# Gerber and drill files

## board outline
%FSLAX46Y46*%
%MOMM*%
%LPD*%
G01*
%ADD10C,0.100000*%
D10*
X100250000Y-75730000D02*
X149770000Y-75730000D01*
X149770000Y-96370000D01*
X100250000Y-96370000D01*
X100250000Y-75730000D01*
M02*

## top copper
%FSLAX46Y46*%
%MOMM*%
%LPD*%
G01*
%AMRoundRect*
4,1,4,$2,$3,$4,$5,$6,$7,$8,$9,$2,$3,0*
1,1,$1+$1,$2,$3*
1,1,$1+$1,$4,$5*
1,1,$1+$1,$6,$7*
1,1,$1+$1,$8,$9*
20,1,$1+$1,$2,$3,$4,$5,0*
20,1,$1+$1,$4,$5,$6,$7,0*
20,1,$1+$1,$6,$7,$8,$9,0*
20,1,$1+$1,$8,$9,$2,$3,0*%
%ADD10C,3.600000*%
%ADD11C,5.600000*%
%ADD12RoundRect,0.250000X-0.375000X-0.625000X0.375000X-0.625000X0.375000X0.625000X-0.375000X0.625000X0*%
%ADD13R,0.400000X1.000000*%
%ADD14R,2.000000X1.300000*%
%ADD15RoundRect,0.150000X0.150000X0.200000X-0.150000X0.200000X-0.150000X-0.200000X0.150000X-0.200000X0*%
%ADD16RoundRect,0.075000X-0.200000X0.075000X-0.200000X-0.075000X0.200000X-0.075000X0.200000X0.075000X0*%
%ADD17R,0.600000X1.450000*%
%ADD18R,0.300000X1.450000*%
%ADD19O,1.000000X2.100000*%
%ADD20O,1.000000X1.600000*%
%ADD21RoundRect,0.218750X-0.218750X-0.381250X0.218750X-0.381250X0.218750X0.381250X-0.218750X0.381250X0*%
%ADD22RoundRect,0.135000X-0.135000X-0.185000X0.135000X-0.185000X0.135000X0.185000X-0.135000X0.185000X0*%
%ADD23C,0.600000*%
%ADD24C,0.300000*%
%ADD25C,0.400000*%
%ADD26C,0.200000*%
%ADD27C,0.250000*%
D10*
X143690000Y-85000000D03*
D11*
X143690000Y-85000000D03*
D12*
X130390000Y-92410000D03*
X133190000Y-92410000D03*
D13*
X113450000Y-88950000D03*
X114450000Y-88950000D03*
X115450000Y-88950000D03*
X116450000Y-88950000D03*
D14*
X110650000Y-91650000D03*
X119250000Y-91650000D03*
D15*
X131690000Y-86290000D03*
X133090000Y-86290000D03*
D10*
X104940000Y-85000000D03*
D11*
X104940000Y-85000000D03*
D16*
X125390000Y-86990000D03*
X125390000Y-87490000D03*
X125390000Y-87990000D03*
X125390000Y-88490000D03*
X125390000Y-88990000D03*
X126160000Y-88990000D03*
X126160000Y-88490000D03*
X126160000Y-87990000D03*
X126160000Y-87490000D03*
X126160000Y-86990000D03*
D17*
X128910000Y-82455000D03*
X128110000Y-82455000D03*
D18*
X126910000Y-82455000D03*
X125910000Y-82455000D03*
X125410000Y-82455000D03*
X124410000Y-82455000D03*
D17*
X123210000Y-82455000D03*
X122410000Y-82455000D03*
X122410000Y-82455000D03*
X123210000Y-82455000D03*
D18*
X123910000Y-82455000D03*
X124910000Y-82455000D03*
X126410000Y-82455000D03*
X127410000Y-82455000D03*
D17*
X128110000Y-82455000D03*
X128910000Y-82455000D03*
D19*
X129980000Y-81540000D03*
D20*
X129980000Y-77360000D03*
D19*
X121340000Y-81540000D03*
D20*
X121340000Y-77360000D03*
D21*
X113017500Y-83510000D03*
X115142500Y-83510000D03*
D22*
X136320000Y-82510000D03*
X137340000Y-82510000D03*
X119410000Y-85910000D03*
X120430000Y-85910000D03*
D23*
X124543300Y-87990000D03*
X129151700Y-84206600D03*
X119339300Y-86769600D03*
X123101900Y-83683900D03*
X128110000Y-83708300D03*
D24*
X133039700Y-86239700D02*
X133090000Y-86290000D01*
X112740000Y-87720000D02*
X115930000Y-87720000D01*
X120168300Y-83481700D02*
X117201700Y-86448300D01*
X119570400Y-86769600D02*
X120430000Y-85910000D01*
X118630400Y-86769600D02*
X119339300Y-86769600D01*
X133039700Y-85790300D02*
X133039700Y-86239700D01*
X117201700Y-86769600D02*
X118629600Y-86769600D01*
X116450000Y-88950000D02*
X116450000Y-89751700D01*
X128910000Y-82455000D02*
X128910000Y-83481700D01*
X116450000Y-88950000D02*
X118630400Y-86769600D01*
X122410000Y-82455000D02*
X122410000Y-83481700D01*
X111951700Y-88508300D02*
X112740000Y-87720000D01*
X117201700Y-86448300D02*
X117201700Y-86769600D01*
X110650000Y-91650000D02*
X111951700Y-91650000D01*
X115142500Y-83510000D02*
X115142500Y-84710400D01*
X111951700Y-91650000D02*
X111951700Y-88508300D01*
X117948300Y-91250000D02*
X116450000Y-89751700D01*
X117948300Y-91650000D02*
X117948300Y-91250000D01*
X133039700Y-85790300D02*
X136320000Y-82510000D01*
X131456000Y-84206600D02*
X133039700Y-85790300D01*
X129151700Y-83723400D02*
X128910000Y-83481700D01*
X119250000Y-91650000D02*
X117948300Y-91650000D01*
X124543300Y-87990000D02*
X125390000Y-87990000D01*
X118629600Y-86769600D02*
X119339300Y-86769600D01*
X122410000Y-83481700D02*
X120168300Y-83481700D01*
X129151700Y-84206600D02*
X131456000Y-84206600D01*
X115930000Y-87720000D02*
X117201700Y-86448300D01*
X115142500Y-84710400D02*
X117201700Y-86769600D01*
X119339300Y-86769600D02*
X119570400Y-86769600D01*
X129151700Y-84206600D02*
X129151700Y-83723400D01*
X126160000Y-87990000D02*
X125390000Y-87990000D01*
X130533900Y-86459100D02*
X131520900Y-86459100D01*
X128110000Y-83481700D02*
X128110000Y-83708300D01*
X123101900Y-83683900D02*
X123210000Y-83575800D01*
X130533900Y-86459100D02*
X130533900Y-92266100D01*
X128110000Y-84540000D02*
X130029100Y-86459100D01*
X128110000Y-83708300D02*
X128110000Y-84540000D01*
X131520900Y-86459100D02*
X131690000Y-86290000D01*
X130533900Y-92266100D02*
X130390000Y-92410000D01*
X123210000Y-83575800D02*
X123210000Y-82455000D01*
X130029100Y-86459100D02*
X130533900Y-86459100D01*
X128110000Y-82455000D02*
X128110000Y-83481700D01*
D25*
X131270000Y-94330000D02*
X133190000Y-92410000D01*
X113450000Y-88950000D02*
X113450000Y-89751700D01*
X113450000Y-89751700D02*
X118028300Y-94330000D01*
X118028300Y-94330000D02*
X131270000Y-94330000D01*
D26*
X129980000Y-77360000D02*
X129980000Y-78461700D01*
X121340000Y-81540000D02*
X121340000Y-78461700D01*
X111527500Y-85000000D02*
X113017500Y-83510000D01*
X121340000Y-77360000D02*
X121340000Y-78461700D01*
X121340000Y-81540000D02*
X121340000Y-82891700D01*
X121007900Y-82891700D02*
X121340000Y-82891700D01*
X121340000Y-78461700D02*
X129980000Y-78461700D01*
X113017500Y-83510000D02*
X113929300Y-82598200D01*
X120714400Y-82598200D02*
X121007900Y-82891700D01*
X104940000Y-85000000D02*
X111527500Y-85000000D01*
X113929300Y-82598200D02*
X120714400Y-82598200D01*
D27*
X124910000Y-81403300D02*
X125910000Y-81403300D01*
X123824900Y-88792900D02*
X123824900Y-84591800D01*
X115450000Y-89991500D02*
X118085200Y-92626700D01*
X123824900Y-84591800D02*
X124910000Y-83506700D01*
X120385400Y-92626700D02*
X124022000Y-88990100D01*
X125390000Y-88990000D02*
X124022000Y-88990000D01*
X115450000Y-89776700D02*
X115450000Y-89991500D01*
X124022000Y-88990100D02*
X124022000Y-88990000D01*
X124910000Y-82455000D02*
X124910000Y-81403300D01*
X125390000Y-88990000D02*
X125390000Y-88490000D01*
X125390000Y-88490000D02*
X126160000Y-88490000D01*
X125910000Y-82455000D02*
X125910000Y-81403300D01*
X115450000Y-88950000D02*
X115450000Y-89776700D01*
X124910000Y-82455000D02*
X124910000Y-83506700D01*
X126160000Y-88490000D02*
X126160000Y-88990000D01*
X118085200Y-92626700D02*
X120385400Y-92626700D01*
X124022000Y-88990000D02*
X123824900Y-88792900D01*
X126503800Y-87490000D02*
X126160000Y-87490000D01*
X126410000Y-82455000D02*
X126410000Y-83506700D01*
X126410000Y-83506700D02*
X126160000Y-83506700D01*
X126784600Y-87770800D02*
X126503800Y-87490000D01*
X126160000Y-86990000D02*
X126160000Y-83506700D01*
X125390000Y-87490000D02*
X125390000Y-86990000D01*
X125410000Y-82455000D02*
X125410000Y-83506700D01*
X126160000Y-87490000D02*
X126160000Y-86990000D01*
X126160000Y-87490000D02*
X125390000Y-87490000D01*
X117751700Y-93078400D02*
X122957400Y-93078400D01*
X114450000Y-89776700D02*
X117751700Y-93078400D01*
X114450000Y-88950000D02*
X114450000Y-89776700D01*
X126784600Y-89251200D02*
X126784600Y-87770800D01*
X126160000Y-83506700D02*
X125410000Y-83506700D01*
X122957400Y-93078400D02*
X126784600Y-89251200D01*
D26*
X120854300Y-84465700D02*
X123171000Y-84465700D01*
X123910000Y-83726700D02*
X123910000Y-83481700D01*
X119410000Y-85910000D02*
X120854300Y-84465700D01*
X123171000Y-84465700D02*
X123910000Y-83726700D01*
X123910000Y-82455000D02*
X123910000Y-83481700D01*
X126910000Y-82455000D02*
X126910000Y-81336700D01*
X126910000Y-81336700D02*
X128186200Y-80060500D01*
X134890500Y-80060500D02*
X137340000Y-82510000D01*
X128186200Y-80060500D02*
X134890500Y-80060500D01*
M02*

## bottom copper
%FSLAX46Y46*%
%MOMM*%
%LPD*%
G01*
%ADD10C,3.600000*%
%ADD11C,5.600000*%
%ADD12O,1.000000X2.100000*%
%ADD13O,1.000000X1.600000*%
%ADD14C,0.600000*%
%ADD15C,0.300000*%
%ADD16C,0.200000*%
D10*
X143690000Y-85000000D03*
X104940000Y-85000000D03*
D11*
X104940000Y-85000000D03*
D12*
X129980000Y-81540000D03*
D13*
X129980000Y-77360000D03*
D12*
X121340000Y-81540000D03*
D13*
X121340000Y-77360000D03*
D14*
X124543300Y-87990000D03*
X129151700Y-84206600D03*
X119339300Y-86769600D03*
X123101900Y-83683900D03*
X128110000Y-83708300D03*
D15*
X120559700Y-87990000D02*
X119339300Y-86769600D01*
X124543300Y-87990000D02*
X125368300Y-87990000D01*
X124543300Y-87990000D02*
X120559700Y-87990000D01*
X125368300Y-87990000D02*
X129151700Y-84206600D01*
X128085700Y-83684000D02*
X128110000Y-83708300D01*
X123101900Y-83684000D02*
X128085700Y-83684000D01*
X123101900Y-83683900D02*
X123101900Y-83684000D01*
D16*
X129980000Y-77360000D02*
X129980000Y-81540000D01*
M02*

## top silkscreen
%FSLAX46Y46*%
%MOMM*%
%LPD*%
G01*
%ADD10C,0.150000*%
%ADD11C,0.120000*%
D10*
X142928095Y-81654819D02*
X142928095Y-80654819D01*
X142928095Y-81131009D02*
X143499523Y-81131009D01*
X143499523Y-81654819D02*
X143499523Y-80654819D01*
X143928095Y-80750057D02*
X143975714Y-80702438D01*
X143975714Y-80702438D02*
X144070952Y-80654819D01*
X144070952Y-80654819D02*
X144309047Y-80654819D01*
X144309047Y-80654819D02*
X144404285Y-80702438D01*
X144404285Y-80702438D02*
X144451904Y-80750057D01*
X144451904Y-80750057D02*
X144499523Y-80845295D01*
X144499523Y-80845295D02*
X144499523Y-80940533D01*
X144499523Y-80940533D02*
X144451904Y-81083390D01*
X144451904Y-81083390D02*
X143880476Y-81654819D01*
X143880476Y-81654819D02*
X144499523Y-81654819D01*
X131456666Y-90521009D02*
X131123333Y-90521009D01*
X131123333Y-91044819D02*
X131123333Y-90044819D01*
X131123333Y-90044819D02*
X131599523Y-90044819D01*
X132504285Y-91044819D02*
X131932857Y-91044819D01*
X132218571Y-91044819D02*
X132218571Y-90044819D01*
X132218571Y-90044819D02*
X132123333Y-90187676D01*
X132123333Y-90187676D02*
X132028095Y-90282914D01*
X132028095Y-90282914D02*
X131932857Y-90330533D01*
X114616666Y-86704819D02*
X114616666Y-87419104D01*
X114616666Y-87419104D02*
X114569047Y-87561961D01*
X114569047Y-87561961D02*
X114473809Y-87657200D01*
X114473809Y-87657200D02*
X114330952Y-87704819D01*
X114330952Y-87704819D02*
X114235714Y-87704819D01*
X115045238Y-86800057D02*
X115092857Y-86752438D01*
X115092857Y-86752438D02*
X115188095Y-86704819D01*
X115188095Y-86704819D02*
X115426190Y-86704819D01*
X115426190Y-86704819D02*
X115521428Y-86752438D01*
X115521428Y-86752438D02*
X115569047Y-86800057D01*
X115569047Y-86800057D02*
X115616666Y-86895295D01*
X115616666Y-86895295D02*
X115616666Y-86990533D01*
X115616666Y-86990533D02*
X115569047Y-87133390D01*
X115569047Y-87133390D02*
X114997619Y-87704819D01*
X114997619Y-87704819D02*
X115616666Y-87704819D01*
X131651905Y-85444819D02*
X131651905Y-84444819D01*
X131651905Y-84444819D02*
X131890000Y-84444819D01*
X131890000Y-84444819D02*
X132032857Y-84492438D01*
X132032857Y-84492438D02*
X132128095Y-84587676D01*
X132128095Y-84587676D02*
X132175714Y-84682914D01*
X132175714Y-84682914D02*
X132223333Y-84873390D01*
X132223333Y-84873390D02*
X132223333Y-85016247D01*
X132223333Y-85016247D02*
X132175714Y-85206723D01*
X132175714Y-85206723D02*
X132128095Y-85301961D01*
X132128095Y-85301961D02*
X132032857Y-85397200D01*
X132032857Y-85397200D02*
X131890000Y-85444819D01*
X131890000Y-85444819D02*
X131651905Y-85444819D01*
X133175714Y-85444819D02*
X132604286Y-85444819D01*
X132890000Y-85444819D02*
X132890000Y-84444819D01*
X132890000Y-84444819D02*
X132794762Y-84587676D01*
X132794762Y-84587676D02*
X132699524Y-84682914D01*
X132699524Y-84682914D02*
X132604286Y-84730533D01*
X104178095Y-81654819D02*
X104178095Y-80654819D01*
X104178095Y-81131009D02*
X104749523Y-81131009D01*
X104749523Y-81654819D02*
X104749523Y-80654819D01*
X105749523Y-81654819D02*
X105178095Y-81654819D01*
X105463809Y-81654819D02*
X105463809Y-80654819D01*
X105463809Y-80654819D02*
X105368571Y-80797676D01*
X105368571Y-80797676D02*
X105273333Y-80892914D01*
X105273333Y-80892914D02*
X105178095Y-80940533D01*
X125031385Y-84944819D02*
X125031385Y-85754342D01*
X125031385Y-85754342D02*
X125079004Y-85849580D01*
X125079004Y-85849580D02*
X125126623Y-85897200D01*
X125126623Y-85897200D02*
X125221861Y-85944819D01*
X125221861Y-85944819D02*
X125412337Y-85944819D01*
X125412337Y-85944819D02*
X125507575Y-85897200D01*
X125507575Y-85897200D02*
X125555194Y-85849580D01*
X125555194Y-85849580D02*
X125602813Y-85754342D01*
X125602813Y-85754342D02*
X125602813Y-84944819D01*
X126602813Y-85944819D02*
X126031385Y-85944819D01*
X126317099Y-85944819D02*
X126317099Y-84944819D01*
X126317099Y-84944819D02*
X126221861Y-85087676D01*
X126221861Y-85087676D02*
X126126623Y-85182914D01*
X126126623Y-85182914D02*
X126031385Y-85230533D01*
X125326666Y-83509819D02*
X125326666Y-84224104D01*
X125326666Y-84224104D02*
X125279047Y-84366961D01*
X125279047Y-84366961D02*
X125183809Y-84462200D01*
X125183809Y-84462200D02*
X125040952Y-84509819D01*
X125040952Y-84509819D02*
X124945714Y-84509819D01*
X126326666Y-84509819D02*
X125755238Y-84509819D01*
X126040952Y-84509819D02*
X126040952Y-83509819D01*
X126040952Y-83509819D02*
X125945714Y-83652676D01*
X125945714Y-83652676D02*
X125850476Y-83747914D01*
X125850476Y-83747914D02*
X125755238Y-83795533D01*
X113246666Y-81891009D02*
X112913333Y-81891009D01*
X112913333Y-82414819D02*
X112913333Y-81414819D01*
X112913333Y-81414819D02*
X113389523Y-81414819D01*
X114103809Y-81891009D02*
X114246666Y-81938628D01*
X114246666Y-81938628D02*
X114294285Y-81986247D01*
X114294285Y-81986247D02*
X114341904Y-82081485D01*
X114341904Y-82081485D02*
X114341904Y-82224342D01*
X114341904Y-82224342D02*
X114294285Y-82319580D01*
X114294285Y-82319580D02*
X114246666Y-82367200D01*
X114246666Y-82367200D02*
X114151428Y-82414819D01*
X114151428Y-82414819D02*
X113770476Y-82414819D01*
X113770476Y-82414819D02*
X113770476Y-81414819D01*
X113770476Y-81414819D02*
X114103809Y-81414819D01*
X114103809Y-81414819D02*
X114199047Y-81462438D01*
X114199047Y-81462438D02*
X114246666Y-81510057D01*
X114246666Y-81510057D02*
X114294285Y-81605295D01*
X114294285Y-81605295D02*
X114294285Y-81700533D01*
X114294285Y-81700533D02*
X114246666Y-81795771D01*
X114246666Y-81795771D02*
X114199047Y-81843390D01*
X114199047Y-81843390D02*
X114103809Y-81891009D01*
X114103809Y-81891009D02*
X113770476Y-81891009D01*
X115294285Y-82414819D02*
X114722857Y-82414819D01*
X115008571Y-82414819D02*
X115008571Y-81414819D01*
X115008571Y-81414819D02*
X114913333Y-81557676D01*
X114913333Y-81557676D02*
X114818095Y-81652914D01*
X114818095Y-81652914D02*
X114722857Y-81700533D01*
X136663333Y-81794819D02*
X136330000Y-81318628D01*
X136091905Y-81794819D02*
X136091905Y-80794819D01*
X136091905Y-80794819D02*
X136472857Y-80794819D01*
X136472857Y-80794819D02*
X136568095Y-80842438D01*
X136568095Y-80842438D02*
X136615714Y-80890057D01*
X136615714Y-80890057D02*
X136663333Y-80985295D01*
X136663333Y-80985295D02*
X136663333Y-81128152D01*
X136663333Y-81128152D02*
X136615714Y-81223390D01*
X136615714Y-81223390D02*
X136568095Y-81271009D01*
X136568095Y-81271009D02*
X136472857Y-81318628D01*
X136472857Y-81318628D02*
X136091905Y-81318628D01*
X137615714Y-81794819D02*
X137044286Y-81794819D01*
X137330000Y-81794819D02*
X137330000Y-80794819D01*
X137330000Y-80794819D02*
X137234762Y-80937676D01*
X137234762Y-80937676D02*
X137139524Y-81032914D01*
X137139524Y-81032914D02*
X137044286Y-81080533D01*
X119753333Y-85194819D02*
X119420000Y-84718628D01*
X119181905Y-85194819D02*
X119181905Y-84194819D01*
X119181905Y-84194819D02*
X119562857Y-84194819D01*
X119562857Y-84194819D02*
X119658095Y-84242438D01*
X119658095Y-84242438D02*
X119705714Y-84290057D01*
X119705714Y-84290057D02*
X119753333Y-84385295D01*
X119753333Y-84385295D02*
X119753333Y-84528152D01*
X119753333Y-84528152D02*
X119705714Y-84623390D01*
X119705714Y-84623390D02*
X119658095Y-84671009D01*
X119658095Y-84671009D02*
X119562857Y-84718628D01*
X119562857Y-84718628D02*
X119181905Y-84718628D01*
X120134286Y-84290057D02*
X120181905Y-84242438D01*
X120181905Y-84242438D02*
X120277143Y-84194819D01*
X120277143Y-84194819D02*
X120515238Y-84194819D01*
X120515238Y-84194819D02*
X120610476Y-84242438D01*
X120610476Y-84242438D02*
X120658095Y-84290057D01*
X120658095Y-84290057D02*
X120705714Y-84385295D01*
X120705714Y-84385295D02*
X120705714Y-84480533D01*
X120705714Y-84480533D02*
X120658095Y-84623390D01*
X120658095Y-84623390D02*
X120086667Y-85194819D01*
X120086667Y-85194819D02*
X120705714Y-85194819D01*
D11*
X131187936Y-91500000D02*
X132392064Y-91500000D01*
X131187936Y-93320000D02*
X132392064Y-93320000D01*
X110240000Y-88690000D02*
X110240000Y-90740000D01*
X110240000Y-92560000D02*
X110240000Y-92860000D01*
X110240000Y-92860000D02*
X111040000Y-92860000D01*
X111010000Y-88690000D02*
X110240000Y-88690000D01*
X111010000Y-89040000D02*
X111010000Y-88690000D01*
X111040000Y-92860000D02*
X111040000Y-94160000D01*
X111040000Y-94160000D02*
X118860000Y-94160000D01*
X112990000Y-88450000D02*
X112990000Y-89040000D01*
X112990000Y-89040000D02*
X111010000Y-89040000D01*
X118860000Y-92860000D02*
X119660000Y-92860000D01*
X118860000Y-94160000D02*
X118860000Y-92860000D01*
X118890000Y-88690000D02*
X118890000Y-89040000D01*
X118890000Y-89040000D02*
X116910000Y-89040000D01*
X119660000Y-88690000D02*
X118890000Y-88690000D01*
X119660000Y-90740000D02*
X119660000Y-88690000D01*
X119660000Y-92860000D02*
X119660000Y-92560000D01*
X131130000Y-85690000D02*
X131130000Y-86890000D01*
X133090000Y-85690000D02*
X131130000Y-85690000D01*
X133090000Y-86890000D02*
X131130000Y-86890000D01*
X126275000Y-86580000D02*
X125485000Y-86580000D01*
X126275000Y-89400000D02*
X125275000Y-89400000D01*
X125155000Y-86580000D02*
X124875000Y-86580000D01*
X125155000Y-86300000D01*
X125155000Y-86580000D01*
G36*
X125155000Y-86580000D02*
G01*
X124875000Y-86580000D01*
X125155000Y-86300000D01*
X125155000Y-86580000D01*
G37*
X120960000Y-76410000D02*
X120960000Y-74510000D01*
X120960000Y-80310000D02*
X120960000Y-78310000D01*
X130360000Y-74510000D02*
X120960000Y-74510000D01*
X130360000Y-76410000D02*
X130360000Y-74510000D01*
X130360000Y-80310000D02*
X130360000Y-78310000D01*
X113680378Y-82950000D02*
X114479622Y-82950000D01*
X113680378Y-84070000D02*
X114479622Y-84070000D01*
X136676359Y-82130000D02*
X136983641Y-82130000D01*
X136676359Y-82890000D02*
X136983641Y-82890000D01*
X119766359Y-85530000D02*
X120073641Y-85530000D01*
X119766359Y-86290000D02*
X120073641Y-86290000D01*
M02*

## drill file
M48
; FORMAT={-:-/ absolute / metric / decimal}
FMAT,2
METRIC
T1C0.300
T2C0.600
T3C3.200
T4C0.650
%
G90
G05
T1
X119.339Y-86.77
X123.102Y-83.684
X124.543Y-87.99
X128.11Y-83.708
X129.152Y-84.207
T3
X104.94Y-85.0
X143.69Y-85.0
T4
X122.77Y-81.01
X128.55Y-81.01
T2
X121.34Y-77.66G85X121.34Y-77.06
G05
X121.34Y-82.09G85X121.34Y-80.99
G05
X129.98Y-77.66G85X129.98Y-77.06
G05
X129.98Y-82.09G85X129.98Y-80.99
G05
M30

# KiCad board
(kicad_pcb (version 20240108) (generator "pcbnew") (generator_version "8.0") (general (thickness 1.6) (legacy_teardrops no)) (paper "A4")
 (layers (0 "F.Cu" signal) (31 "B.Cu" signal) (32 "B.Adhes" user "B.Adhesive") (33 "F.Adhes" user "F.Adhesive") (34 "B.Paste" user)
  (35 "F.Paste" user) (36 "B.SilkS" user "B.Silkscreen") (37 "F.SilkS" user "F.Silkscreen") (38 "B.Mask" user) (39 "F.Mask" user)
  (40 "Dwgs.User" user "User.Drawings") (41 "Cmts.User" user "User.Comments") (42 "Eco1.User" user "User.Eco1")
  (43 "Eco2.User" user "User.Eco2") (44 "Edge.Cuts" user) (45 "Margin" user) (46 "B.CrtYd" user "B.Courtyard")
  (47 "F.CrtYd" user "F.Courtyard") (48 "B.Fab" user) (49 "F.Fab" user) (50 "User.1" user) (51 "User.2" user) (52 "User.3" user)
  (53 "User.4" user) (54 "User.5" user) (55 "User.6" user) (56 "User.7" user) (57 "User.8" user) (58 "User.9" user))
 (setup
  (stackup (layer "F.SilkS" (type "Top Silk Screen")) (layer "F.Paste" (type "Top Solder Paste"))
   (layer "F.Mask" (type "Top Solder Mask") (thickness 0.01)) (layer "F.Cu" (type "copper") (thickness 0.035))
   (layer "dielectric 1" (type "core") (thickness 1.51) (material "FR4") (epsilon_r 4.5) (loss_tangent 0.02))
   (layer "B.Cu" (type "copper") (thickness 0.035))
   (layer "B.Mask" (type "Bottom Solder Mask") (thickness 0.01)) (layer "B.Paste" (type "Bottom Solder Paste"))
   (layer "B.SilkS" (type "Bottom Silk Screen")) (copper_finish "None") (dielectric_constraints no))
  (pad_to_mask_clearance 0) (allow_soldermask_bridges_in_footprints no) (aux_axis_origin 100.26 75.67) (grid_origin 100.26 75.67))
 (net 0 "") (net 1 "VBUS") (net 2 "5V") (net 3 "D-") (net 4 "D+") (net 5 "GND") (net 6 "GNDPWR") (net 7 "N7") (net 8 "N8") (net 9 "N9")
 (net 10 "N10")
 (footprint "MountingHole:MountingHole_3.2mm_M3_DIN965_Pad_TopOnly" (layer "F.Cu") (at 143.69 85)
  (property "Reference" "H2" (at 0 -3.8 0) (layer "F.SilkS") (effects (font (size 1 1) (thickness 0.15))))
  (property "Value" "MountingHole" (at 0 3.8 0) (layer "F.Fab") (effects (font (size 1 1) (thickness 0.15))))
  (pad "1" thru_hole circle (at 0 0) (size 3.6 3.6) (drill 3.2) (layers "*.Cu" "*.Mask") (remove_unused_layers no))
  (pad "1" connect circle (at 0 0) (size 5.6 5.6) (layers "F.Cu" "F.Mask")))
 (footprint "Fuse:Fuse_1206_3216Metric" (layer "F.Cu") (at 131.79 92.41)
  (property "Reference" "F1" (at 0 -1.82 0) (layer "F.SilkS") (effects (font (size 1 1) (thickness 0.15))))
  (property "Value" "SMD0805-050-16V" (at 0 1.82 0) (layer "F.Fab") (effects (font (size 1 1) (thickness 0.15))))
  (fp_line (start -0.602064 -0.91) (end 0.602064 -0.91) (stroke (width 0.12) (type solid)) (layer "F.SilkS"))
  (fp_line (start -0.602064 0.91) (end 0.602064 0.91) (stroke (width 0.12) (type solid)) (layer "F.SilkS"))
  (pad "1" smd roundrect (at -1.4 0) (size 1.25 1.75) (layers "F.Cu" "F.Paste" "F.Mask") (roundrect_rratio 0.2) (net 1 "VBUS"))
  (pad "2" smd roundrect (at 1.4 0) (size 1.25 1.75) (layers "F.Cu" "F.Paste" "F.Mask") (roundrect_rratio 0.2) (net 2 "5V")))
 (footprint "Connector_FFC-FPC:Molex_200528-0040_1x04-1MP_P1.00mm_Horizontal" (layer "F.Cu") (at 114.95 89.86)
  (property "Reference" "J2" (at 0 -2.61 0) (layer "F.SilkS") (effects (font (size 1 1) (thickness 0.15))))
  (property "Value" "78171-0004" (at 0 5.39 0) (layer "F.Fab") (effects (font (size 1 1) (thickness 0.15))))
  (fp_line (start -4.71 -1.17) (end -4.71 0.88) (stroke (width 0.12) (type solid)) (layer "F.SilkS"))
  (fp_line (start -4.71 2.7) (end -4.71 3) (stroke (width 0.12) (type solid)) (layer "F.SilkS"))
  (fp_line (start -4.71 3) (end -3.91 3) (stroke (width 0.12) (type solid)) (layer "F.SilkS"))
  (fp_line (start -3.94 -1.17) (end -4.71 -1.17) (stroke (width 0.12) (type solid)) (layer "F.SilkS"))
  (fp_line (start -3.94 -0.82) (end -3.94 -1.17) (stroke (width 0.12) (type solid)) (layer "F.SilkS"))
  (fp_line (start -3.91 3) (end -3.91 4.3) (stroke (width 0.12) (type solid)) (layer "F.SilkS"))
  (fp_line (start -3.91 4.3) (end 3.91 4.3) (stroke (width 0.12) (type solid)) (layer "F.SilkS"))
  (fp_line (start -1.96 -1.41) (end -1.96 -0.82) (stroke (width 0.12) (type solid)) (layer "F.SilkS"))
  (fp_line (start -1.96 -0.82) (end -3.94 -0.82) (stroke (width 0.12) (type solid)) (layer "F.SilkS"))
  (fp_line (start 3.91 3) (end 4.71 3) (stroke (width 0.12) (type solid)) (layer "F.SilkS"))
  (fp_line (start 3.91 4.3) (end 3.91 3) (stroke (width 0.12) (type solid)) (layer "F.SilkS"))
  (fp_line (start 3.94 -1.17) (end 3.94 -0.82) (stroke (width 0.12) (type solid)) (layer "F.SilkS"))
  (fp_line (start 3.94 -0.82) (end 1.96 -0.82) (stroke (width 0.12) (type solid)) (layer "F.SilkS"))
  (fp_line (start 4.71 -1.17) (end 3.94 -1.17) (stroke (width 0.12) (type solid)) (layer "F.SilkS"))
  (fp_line (start 4.71 0.88) (end 4.71 -1.17) (stroke (width 0.12) (type solid)) (layer "F.SilkS"))
  (fp_line (start 4.71 3) (end 4.71 2.7) (stroke (width 0.12) (type solid)) (layer "F.SilkS"))
  (pad "1" smd rect (at -1.5 -0.91) (size 0.4 1) (layers "F.Cu" "F.Paste" "F.Mask") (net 2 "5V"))
  (pad "2" smd rect (at -0.5 -0.91) (size 0.4 1) (layers "F.Cu" "F.Paste" "F.Mask") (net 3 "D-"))
  (pad "3" smd rect (at 0.5 -0.91) (size 0.4 1) (layers "F.Cu" "F.Paste" "F.Mask") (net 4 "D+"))
  (pad "4" smd rect (at 1.5 -0.91) (size 0.4 1) (layers "F.Cu" "F.Paste" "F.Mask") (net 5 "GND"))
  (pad "MP" smd rect (at -4.3 1.79) (size 2 1.3) (layers "F.Cu" "F.Paste" "F.Mask") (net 5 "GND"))
  (pad "MP" smd rect (at 4.3 1.79) (size 2 1.3) (layers "F.Cu" "F.Paste" "F.Mask") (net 5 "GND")))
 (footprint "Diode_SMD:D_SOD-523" (layer "F.Cu") (at 132.39 86.29)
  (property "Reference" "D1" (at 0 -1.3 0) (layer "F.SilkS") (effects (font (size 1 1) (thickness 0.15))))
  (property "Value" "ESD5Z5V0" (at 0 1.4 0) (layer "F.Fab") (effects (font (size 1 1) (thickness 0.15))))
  (fp_line (start -1.26 -0.6) (end -1.26 0.6) (stroke (width 0.12) (type solid)) (layer "F.SilkS"))
  (fp_line (start 0.7 -0.6) (end -1.26 -0.6) (stroke (width 0.12) (type solid)) (layer "F.SilkS"))
  (fp_line (start 0.7 0.6) (end -1.26 0.6) (stroke (width 0.12) (type solid)) (layer "F.SilkS"))
  (pad "1" smd roundrect (at -0.7 0 180) (size 0.6 0.7) (layers "F.Cu" "F.Paste" "F.Mask") (roundrect_rratio 0.25) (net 1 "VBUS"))
  (pad "2" smd roundrect (at 0.7 0 180) (size 0.6 0.7) (layers "F.Cu" "F.Paste" "F.Mask") (roundrect_rratio 0.25) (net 5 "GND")))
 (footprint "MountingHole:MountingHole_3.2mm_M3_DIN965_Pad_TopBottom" (layer "F.Cu") (at 104.94 85)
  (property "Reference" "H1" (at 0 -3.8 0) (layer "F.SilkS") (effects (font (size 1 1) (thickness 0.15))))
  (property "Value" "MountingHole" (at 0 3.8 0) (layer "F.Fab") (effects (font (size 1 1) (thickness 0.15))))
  (pad "1" thru_hole circle (at 0 0) (size 3.6 3.6) (drill 3.2) (layers "*.Cu" "*.Mask") (remove_unused_layers no) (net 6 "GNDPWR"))
  (pad "1" connect circle (at 0 0) (size 5.6 5.6) (layers "F.Cu" "F.Mask") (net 6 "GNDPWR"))
  (pad "1" connect circle (at 0 0) (size 5.6 5.6) (layers "B.Cu" "B.Mask") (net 6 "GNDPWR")))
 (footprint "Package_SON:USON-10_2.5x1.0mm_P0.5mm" (layer "F.Cu") (at 125.775 87.99)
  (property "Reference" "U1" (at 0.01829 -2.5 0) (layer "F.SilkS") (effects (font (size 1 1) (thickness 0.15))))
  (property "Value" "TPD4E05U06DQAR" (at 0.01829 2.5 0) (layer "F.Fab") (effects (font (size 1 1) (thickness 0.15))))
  (fp_line (start 0.5 -1.41) (end -0.29 -1.41) (stroke (width 0.12) (type solid)) (layer "F.SilkS"))
  (fp_line (start 0.5 1.41) (end -0.5 1.41) (stroke (width 0.12) (type solid)) (layer "F.SilkS"))
  (fp_poly
   (pts (xy -0.62 -1.41) (xy -0.9 -1.41) (xy -0.62 -1.69) (xy -0.62 -1.41)) (stroke (width 0.12) (type solid)) (fill solid)
   (layer "F.SilkS"))
  (pad "1" smd roundrect (at -0.385 -1 270) (size 0.3 0.55) (layers "F.Cu" "F.Paste" "F.Mask") (roundrect_rratio 0.25) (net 3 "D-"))
  (pad "2" smd roundrect (at -0.385 -0.5 270) (size 0.3 0.55) (layers "F.Cu" "F.Paste" "F.Mask") (roundrect_rratio 0.25) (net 3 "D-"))
  (pad "3" smd roundrect (at -0.385 0 270) (size 0.3 0.55) (layers "F.Cu" "F.Paste" "F.Mask") (roundrect_rratio 0.25) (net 5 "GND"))
  (pad "4" smd roundrect (at -0.385 0.5 270) (size 0.3 0.55) (layers "F.Cu" "F.Paste" "F.Mask") (roundrect_rratio 0.25) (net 4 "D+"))
  (pad "5" smd roundrect (at -0.385 1 270) (size 0.3 0.55) (layers "F.Cu" "F.Paste" "F.Mask") (roundrect_rratio 0.25) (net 4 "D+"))
  (pad "6" smd roundrect (at 0.385 1 270) (size 0.3 0.55) (layers "F.Cu" "F.Paste" "F.Mask") (roundrect_rratio 0.25) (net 4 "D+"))
  (pad "7" smd roundrect (at 0.385 0.5 270) (size 0.3 0.55) (layers "F.Cu" "F.Paste" "F.Mask") (roundrect_rratio 0.25) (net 4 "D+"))
  (pad "8" smd roundrect (at 0.385 0 270) (size 0.3 0.55) (layers "F.Cu" "F.Paste" "F.Mask") (roundrect_rratio 0.25) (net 5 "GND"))
  (pad "9" smd roundrect (at 0.385 -0.5 270) (size 0.3 0.55) (layers "F.Cu" "F.Paste" "F.Mask") (roundrect_rratio 0.25) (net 3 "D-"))
  (pad "10" smd roundrect (at 0.385 -1 270) (size 0.3 0.55) (layers "F.Cu" "F.Paste" "F.Mask") (roundrect_rratio 0.25) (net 3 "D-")))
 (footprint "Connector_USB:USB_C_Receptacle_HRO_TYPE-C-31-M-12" (layer "F.Cu") (at 125.66 78.41 180)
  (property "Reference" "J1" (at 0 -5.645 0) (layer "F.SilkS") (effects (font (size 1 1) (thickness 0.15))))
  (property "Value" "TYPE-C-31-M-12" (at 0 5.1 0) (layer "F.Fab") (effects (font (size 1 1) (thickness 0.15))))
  (fp_line (start 4.7 2) (end 4.7 3.9) (stroke (width 0.12) (type solid)) (layer "F.SilkS"))
  (fp_line (start 4.7 -1.9) (end 4.7 0.1) (stroke (width 0.12) (type solid)) (layer "F.SilkS"))
  (fp_line (start -4.7 3.9) (end 4.7 3.9) (stroke (width 0.12) (type solid)) (layer "F.SilkS"))
  (fp_line (start -4.7 2) (end -4.7 3.9) (stroke (width 0.12) (type solid)) (layer "F.SilkS"))
  (fp_line (start -4.7 -1.9) (end -4.7 0.1) (stroke (width 0.12) (type solid)) (layer "F.SilkS"))
  (pad "" np_thru_hole circle (at -2.89 -2.6 180) (size 0.65 0.65) (drill 0.65) (layers "*.Cu" "*.Mask"))
  (pad "" np_thru_hole circle (at 2.89 -2.6 180) (size 0.65 0.65) (drill 0.65) (layers "*.Cu" "*.Mask"))
  (pad "A1" smd rect (at -3.25 -4.045 180) (size 0.6 1.45) (layers "F.Cu" "F.Paste" "F.Mask") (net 5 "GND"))
  (pad "A4" smd rect (at -2.45 -4.045 180) (size 0.6 1.45) (layers "F.Cu" "F.Paste" "F.Mask") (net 1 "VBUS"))
  (pad "A5" smd rect (at -1.25 -4.045 180) (size 0.3 1.45) (layers "F.Cu" "F.Paste" "F.Mask") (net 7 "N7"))
  (pad "A6" smd rect (at -0.25 -4.045 180) (size 0.3 1.45) (layers "F.Cu" "F.Paste" "F.Mask") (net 4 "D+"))
  (pad "A7" smd rect (at 0.25 -4.045 180) (size 0.3 1.45) (layers "F.Cu" "F.Paste" "F.Mask") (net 3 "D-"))
  (pad "A8" smd rect (at 1.25 -4.045 180) (size 0.3 1.45) (layers "F.Cu" "F.Paste" "F.Mask") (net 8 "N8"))
  (pad "A9" smd rect (at 2.45 -4.045 180) (size 0.6 1.45) (layers "F.Cu" "F.Paste" "F.Mask") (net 1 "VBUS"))
  (pad "A12" smd rect (at 3.25 -4.045 180) (size 0.6 1.45) (layers "F.Cu" "F.Paste" "F.Mask") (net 5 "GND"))
  (pad "B1" smd rect (at 3.25 -4.045 180) (size 0.6 1.45) (layers "F.Cu" "F.Paste" "F.Mask") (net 5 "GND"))
  (pad "B4" smd rect (at 2.45 -4.045 180) (size 0.6 1.45) (layers "F.Cu" "F.Paste" "F.Mask") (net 1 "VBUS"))
  (pad "B5" smd rect (at 1.75 -4.045 180) (size 0.3 1.45) (layers "F.Cu" "F.Paste" "F.Mask") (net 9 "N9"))
  (pad "B6" smd rect (at 0.75 -4.045 180) (size 0.3 1.45) (layers "F.Cu" "F.Paste" "F.Mask") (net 4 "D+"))
  (pad "B7" smd rect (at -0.75 -4.045 180) (size 0.3 1.45) (layers "F.Cu" "F.Paste" "F.Mask") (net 3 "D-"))
  (pad "B8" smd rect (at -1.75 -4.045 180) (size 0.3 1.45) (layers "F.Cu" "F.Paste" "F.Mask") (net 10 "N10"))
  (pad "B9" smd rect (at -2.45 -4.045 180) (size 0.6 1.45) (layers "F.Cu" "F.Paste" "F.Mask") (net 1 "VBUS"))
  (pad "B12" smd rect (at -3.25 -4.045 180) (size 0.6 1.45) (layers "F.Cu" "F.Paste" "F.Mask") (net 5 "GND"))
  (pad "S1" thru_hole oval (at -4.32 -3.13 180) (size 1 2.1) (drill oval 0.6 1.7) (layers "*.Cu" "*.Mask") (remove_unused_layers no)
   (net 6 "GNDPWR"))
  (pad "S1" thru_hole oval (at -4.32 1.05 180) (size 1 1.6) (drill oval 0.6 1.2) (layers "*.Cu" "*.Mask") (remove_unused_layers no)
   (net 6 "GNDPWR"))
  (pad "S1" thru_hole oval (at 4.32 -3.13 180) (size 1 2.1) (drill oval 0.6 1.7) (layers "*.Cu" "*.Mask") (remove_unused_layers no)
   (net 6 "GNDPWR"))
  (pad "S1" thru_hole oval (at 4.32 1.05 180) (size 1 1.6) (drill oval 0.6 1.2) (layers "*.Cu" "*.Mask") (remove_unused_layers no)
   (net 6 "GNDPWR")))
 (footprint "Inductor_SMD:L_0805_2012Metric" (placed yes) (layer "F.Cu") (at 114.08 83.51)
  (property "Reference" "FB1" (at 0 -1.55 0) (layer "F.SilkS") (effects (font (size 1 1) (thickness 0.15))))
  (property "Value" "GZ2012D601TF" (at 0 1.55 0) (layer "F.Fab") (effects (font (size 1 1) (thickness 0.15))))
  (fp_line (start -0.399622 -0.56) (end 0.399622 -0.56) (stroke (width 0.12) (type solid)) (layer "F.SilkS"))
  (fp_line (start -0.399622 0.56) (end 0.399622 0.56) (stroke (width 0.12) (type solid)) (layer "F.SilkS"))
  (pad "1" smd roundrect (at -1.0625 0) (size 0.875 1.2) (layers "F.Cu" "F.Paste" "F.Mask") (roundrect_rratio 0.25) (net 6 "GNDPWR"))
  (pad "2" smd roundrect (at 1.0625 0) (size 0.875 1.2) (layers "F.Cu" "F.Paste" "F.Mask") (roundrect_rratio 0.25) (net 5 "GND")))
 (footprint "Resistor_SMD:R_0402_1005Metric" (layer "F.Cu") (at 136.83 82.51)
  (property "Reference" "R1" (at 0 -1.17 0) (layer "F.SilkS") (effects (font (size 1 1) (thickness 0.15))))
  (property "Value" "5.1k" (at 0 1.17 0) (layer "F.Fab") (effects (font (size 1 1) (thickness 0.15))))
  (fp_line (start -0.153641 -0.38) (end 0.153641 -0.38) (stroke (width 0.12) (type solid)) (layer "F.SilkS"))
  (fp_line (start -0.153641 0.38) (end 0.153641 0.38) (stroke (width 0.12) (type solid)) (layer "F.SilkS"))
  (pad "1" smd roundrect (at -0.51 0) (size 0.54 0.64) (layers "F.Cu" "F.Paste" "F.Mask") (roundrect_rratio 0.25) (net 5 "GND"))
  (pad "2" smd roundrect (at 0.51 0) (size 0.54 0.64) (layers "F.Cu" "F.Paste" "F.Mask") (roundrect_rratio 0.25) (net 7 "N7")))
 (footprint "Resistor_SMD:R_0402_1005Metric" (layer "F.Cu") (at 119.92 85.91)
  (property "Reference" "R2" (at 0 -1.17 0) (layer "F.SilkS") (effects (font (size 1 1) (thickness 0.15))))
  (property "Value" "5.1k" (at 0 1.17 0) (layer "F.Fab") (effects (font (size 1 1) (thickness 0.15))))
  (fp_line (start -0.153641 -0.38) (end 0.153641 -0.38) (stroke (width 0.12) (type solid)) (layer "F.SilkS"))
  (fp_line (start -0.153641 0.38) (end 0.153641 0.38) (stroke (width 0.12) (type solid)) (layer "F.SilkS"))
  (pad "1" smd roundrect (at -0.51 0) (size 0.54 0.64) (layers "F.Cu" "F.Paste" "F.Mask") (roundrect_rratio 0.25) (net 9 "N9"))
  (pad "2" smd roundrect (at 0.51 0) (size 0.54 0.64) (layers "F.Cu" "F.Paste" "F.Mask") (roundrect_rratio 0.25) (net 5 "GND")))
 (gr_rect (start 100.25 75.73) (end 149.77 96.37) (stroke (width 0.1) (type default)) (fill none) (layer "Edge.Cuts"))
 (segment (start 133.0397 86.2397) (end 133.09 86.29) (width 0.3) (layer "F.Cu") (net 5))
 (segment (start 112.74 87.72) (end 115.93 87.72) (width 0.3) (layer "F.Cu") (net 5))
 (segment (start 120.1683 83.4817) (end 117.2017 86.4483) (width 0.3) (layer "F.Cu") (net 5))
 (segment (start 119.5704 86.7696) (end 120.43 85.91) (width 0.3) (layer "F.Cu") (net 5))
 (segment (start 118.6304 86.7696) (end 119.3393 86.7696) (width 0.3) (layer "F.Cu") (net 5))
 (segment (start 133.0397 85.7903) (end 133.0397 86.2397) (width 0.3) (layer "F.Cu") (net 5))
 (segment (start 117.2017 86.7696) (end 118.6296 86.7696) (width 0.3) (layer "F.Cu") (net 5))
 (segment (start 116.45 88.95) (end 116.45 89.7517) (width 0.3) (layer "F.Cu") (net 5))
 (segment (start 128.91 82.455) (end 128.91 83.4817) (width 0.3) (layer "F.Cu") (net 5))
 (segment (start 116.45 88.95) (end 118.6304 86.7696) (width 0.3) (layer "F.Cu") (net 5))
 (segment (start 122.41 82.455) (end 122.41 83.4817) (width 0.3) (layer "F.Cu") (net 5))
 (segment (start 111.9517 88.5083) (end 112.74 87.72) (width 0.3) (layer "F.Cu") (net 5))
 (segment (start 117.2017 86.4483) (end 117.2017 86.7696) (width 0.3) (layer "F.Cu") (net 5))
 (segment (start 110.65 91.65) (end 111.9517 91.65) (width 0.3) (layer "F.Cu") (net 5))
 (segment (start 115.1425 83.51) (end 115.1425 84.7104) (width 0.3) (layer "F.Cu") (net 5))
 (segment (start 111.9517 91.65) (end 111.9517 88.5083) (width 0.3) (layer "F.Cu") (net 5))
 (segment (start 117.9483 91.25) (end 116.45 89.7517) (width 0.3) (layer "F.Cu") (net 5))
 (segment (start 117.9483 91.65) (end 117.9483 91.25) (width 0.3) (layer "F.Cu") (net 5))
 (segment (start 133.0397 85.7903) (end 136.32 82.51) (width 0.3) (layer "F.Cu") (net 5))
 (segment (start 131.456 84.2066) (end 133.0397 85.7903) (width 0.3) (layer "F.Cu") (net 5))
 (segment (start 129.1517 83.7234) (end 128.91 83.4817) (width 0.3) (layer "F.Cu") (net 5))
 (segment (start 119.25 91.65) (end 117.9483 91.65) (width 0.3) (layer "F.Cu") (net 5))
 (segment (start 124.5433 87.99) (end 125.39 87.99) (width 0.3) (layer "F.Cu") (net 5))
 (segment (start 118.6296 86.7696) (end 119.3393 86.7696) (width 0.3) (layer "F.Cu") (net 5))
 (segment (start 122.41 83.4817) (end 120.1683 83.4817) (width 0.3) (layer "F.Cu") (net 5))
 (segment (start 129.1517 84.2066) (end 131.456 84.2066) (width 0.3) (layer "F.Cu") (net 5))
 (segment (start 115.93 87.72) (end 117.2017 86.4483) (width 0.3) (layer "F.Cu") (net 5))
 (segment (start 115.1425 84.7104) (end 117.2017 86.7696) (width 0.3) (layer "F.Cu") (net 5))
 (segment (start 119.3393 86.7696) (end 119.5704 86.7696) (width 0.3) (layer "F.Cu") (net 5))
 (segment (start 129.1517 84.2066) (end 129.1517 83.7234) (width 0.3) (layer "F.Cu") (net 5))
 (segment (start 126.16 87.99) (end 125.39 87.99) (width 0.3) (layer "F.Cu") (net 5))
 (via (at 124.5433 87.99) (size 0.6) (drill 0.3) (layers "F.Cu" "B.Cu") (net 5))
 (via (at 129.1517 84.2066) (size 0.6) (drill 0.3) (layers "F.Cu" "B.Cu") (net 5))
 (via (at 119.3393 86.7696) (size 0.6) (drill 0.3) (layers "F.Cu" "B.Cu") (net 5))
 (segment (start 120.5597 87.99) (end 119.3393 86.7696) (width 0.3) (layer "B.Cu") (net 5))
 (segment (start 124.5433 87.99) (end 125.3683 87.99) (width 0.3) (layer "B.Cu") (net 5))
 (segment (start 124.5433 87.99) (end 120.5597 87.99) (width 0.3) (layer "B.Cu") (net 5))
 (segment (start 125.3683 87.99) (end 129.1517 84.2066) (width 0.3) (layer "B.Cu") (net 5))
 (segment (start 130.5339 86.4591) (end 131.5209 86.4591) (width 0.3) (layer "F.Cu") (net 1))
 (segment (start 128.11 83.4817) (end 128.11 83.7083) (width 0.3) (layer "F.Cu") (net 1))
 (segment (start 123.1019 83.6839) (end 123.21 83.5758) (width 0.3) (layer "F.Cu") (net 1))
 (segment (start 130.5339 86.4591) (end 130.5339 92.2661) (width 0.3) (layer "F.Cu") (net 1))
 (segment (start 128.11 84.54) (end 130.0291 86.4591) (width 0.3) (layer "F.Cu") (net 1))
 (segment (start 128.11 83.7083) (end 128.11 84.54) (width 0.3) (layer "F.Cu") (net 1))
 (segment (start 131.5209 86.4591) (end 131.69 86.29) (width 0.3) (layer "F.Cu") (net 1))
 (segment (start 130.5339 92.2661) (end 130.39 92.41) (width 0.3) (layer "F.Cu") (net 1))
 (segment (start 123.21 83.5758) (end 123.21 82.455) (width 0.3) (layer "F.Cu") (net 1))
 (segment (start 130.0291 86.4591) (end 130.5339 86.4591) (width 0.3) (layer "F.Cu") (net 1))
 (segment (start 128.11 82.455) (end 128.11 83.4817) (width 0.3) (layer "F.Cu") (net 1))
 (via (at 123.1019 83.6839) (size 0.6) (drill 0.3) (layers "F.Cu" "B.Cu") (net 1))
 (via (at 128.11 83.7083) (size 0.6) (drill 0.3) (layers "F.Cu" "B.Cu") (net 1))
 (segment (start 128.0857 83.684) (end 128.11 83.7083) (width 0.3) (layer "B.Cu") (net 1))
 (segment (start 123.1019 83.684) (end 128.0857 83.684) (width 0.3) (layer "B.Cu") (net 1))
 (segment (start 123.1019 83.6839) (end 123.1019 83.684) (width 0.3) (layer "B.Cu") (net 1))
 (segment (start 131.27 94.33) (end 133.19 92.41) (width 0.4) (layer "F.Cu") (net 2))
 (segment (start 113.45 88.95) (end 113.45 89.7517) (width 0.4) (layer "F.Cu") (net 2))
 (segment (start 113.45 89.7517) (end 118.0283 94.33) (width 0.4) (layer "F.Cu") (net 2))
 (segment (start 118.0283 94.33) (end 131.27 94.33) (width 0.4) (layer "F.Cu") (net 2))
 (segment (start 129.98 77.36) (end 129.98 78.4617) (width 0.2) (layer "F.Cu") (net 6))
 (segment (start 121.34 81.54) (end 121.34 78.4617) (width 0.2) (layer "F.Cu") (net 6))
 (segment (start 111.5275 85) (end 113.0175 83.51) (width 0.2) (layer "F.Cu") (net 6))
 (segment (start 121.34 77.36) (end 121.34 78.4617) (width 0.2) (layer "F.Cu") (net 6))
 (segment (start 121.34 81.54) (end 121.34 82.8917) (width 0.2) (layer "F.Cu") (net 6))
 (segment (start 121.0079 82.8917) (end 121.34 82.8917) (width 0.2) (layer "F.Cu") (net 6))
 (segment (start 121.34 78.4617) (end 129.98 78.4617) (width 0.2) (layer "F.Cu") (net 6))
 (segment (start 113.0175 83.51) (end 113.9293 82.5982) (width 0.2) (layer "F.Cu") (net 6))
 (segment (start 120.7144 82.5982) (end 121.0079 82.8917) (width 0.2) (layer "F.Cu") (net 6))
 (segment (start 104.94 85) (end 111.5275 85) (width 0.2) (layer "F.Cu") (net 6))
 (segment (start 113.9293 82.5982) (end 120.7144 82.5982) (width 0.2) (layer "F.Cu") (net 6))
 (segment (start 129.98 77.36) (end 129.98 81.54) (width 0.2) (layer "B.Cu") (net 6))
 (segment (start 124.91 81.4033) (end 125.91 81.4033) (width 0.25) (layer "F.Cu") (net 4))
 (segment (start 123.8249 88.7929) (end 123.8249 84.5918) (width 0.25) (layer "F.Cu") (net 4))
 (segment (start 115.45 89.9915) (end 118.0852 92.6267) (width 0.25) (layer "F.Cu") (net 4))
 (segment (start 123.8249 84.5918) (end 124.91 83.5067) (width 0.25) (layer "F.Cu") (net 4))
 (segment (start 120.3854 92.6267) (end 124.022 88.9901) (width 0.25) (layer "F.Cu") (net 4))
 (segment (start 125.39 88.99) (end 124.022 88.99) (width 0.25) (layer "F.Cu") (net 4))
 (segment (start 115.45 89.7767) (end 115.45 89.9915) (width 0.25) (layer "F.Cu") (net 4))
 (segment (start 124.022 88.9901) (end 124.022 88.99) (width 0.25) (layer "F.Cu") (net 4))
 (segment (start 124.91 82.455) (end 124.91 81.4033) (width 0.25) (layer "F.Cu") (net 4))
 (segment (start 125.39 88.99) (end 125.39 88.49) (width 0.25) (layer "F.Cu") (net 4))
 (segment (start 125.39 88.49) (end 126.16 88.49) (width 0.25) (layer "F.Cu") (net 4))
 (segment (start 125.91 82.455) (end 125.91 81.4033) (width 0.25) (layer "F.Cu") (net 4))
 (segment (start 115.45 88.95) (end 115.45 89.7767) (width 0.25) (layer "F.Cu") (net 4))
 (segment (start 124.91 82.455) (end 124.91 83.5067) (width 0.25) (layer "F.Cu") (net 4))
 (segment (start 126.16 88.49) (end 126.16 88.99) (width 0.25) (layer "F.Cu") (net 4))
 (segment (start 118.0852 92.6267) (end 120.3854 92.6267) (width 0.25) (layer "F.Cu") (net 4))
 (segment (start 124.022 88.99) (end 123.8249 88.7929) (width 0.25) (layer "F.Cu") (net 4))
 (segment (start 126.5038 87.49) (end 126.16 87.49) (width 0.25) (layer "F.Cu") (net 3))
 (segment (start 126.41 82.455) (end 126.41 83.5067) (width 0.25) (layer "F.Cu") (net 3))
 (segment (start 126.41 83.5067) (end 126.16 83.5067) (width 0.25) (layer "F.Cu") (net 3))
 (segment (start 126.7846 87.7708) (end 126.5038 87.49) (width 0.25) (layer "F.Cu") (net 3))
 (segment (start 126.16 86.99) (end 126.16 83.5067) (width 0.25) (layer "F.Cu") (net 3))
 (segment (start 125.39 87.49) (end 125.39 86.99) (width 0.25) (layer "F.Cu") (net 3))
 (segment (start 125.41 82.455) (end 125.41 83.5067) (width 0.25) (layer "F.Cu") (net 3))
 (segment (start 126.16 87.49) (end 126.16 86.99) (width 0.25) (layer "F.Cu") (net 3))
 (segment (start 126.16 87.49) (end 125.39 87.49) (width 0.25) (layer "F.Cu") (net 3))
 (segment (start 117.7517 93.0784) (end 122.9574 93.0784) (width 0.25) (layer "F.Cu") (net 3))
 (segment (start 114.45 89.7767) (end 117.7517 93.0784) (width 0.25) (layer "F.Cu") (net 3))
 (segment (start 114.45 88.95) (end 114.45 89.7767) (width 0.25) (layer "F.Cu") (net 3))
 (segment (start 126.7846 89.2512) (end 126.7846 87.7708) (width 0.25) (layer "F.Cu") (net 3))
 (segment (start 126.16 83.5067) (end 125.41 83.5067) (width 0.25) (layer "F.Cu") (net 3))
 (segment (start 122.9574 93.0784) (end 126.7846 89.2512) (width 0.25) (layer "F.Cu") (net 3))
 (segment (start 120.8543 84.4657) (end 123.171 84.4657) (width 0.2) (layer "F.Cu") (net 9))
 (segment (start 123.91 83.7267) (end 123.91 83.4817) (width 0.2) (layer "F.Cu") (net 9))
 (segment (start 119.41 85.91) (end 120.8543 84.4657) (width 0.2) (layer "F.Cu") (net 9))
 (segment (start 123.171 84.4657) (end 123.91 83.7267) (width 0.2) (layer "F.Cu") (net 9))
 (segment (start 123.91 82.455) (end 123.91 83.4817) (width 0.2) (layer "F.Cu") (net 9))
 (segment (start 126.91 82.455) (end 126.91 81.3367) (width 0.2) (layer "F.Cu") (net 7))
 (segment (start 126.91 81.3367) (end 128.1862 80.0605) (width 0.2) (layer "F.Cu") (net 7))
 (segment (start 134.8905 80.0605) (end 137.34 82.51) (width 0.2) (layer "F.Cu") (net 7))
 (segment (start 128.1862 80.0605) (end 134.8905 80.0605) (width 0.2) (layer "F.Cu") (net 7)))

